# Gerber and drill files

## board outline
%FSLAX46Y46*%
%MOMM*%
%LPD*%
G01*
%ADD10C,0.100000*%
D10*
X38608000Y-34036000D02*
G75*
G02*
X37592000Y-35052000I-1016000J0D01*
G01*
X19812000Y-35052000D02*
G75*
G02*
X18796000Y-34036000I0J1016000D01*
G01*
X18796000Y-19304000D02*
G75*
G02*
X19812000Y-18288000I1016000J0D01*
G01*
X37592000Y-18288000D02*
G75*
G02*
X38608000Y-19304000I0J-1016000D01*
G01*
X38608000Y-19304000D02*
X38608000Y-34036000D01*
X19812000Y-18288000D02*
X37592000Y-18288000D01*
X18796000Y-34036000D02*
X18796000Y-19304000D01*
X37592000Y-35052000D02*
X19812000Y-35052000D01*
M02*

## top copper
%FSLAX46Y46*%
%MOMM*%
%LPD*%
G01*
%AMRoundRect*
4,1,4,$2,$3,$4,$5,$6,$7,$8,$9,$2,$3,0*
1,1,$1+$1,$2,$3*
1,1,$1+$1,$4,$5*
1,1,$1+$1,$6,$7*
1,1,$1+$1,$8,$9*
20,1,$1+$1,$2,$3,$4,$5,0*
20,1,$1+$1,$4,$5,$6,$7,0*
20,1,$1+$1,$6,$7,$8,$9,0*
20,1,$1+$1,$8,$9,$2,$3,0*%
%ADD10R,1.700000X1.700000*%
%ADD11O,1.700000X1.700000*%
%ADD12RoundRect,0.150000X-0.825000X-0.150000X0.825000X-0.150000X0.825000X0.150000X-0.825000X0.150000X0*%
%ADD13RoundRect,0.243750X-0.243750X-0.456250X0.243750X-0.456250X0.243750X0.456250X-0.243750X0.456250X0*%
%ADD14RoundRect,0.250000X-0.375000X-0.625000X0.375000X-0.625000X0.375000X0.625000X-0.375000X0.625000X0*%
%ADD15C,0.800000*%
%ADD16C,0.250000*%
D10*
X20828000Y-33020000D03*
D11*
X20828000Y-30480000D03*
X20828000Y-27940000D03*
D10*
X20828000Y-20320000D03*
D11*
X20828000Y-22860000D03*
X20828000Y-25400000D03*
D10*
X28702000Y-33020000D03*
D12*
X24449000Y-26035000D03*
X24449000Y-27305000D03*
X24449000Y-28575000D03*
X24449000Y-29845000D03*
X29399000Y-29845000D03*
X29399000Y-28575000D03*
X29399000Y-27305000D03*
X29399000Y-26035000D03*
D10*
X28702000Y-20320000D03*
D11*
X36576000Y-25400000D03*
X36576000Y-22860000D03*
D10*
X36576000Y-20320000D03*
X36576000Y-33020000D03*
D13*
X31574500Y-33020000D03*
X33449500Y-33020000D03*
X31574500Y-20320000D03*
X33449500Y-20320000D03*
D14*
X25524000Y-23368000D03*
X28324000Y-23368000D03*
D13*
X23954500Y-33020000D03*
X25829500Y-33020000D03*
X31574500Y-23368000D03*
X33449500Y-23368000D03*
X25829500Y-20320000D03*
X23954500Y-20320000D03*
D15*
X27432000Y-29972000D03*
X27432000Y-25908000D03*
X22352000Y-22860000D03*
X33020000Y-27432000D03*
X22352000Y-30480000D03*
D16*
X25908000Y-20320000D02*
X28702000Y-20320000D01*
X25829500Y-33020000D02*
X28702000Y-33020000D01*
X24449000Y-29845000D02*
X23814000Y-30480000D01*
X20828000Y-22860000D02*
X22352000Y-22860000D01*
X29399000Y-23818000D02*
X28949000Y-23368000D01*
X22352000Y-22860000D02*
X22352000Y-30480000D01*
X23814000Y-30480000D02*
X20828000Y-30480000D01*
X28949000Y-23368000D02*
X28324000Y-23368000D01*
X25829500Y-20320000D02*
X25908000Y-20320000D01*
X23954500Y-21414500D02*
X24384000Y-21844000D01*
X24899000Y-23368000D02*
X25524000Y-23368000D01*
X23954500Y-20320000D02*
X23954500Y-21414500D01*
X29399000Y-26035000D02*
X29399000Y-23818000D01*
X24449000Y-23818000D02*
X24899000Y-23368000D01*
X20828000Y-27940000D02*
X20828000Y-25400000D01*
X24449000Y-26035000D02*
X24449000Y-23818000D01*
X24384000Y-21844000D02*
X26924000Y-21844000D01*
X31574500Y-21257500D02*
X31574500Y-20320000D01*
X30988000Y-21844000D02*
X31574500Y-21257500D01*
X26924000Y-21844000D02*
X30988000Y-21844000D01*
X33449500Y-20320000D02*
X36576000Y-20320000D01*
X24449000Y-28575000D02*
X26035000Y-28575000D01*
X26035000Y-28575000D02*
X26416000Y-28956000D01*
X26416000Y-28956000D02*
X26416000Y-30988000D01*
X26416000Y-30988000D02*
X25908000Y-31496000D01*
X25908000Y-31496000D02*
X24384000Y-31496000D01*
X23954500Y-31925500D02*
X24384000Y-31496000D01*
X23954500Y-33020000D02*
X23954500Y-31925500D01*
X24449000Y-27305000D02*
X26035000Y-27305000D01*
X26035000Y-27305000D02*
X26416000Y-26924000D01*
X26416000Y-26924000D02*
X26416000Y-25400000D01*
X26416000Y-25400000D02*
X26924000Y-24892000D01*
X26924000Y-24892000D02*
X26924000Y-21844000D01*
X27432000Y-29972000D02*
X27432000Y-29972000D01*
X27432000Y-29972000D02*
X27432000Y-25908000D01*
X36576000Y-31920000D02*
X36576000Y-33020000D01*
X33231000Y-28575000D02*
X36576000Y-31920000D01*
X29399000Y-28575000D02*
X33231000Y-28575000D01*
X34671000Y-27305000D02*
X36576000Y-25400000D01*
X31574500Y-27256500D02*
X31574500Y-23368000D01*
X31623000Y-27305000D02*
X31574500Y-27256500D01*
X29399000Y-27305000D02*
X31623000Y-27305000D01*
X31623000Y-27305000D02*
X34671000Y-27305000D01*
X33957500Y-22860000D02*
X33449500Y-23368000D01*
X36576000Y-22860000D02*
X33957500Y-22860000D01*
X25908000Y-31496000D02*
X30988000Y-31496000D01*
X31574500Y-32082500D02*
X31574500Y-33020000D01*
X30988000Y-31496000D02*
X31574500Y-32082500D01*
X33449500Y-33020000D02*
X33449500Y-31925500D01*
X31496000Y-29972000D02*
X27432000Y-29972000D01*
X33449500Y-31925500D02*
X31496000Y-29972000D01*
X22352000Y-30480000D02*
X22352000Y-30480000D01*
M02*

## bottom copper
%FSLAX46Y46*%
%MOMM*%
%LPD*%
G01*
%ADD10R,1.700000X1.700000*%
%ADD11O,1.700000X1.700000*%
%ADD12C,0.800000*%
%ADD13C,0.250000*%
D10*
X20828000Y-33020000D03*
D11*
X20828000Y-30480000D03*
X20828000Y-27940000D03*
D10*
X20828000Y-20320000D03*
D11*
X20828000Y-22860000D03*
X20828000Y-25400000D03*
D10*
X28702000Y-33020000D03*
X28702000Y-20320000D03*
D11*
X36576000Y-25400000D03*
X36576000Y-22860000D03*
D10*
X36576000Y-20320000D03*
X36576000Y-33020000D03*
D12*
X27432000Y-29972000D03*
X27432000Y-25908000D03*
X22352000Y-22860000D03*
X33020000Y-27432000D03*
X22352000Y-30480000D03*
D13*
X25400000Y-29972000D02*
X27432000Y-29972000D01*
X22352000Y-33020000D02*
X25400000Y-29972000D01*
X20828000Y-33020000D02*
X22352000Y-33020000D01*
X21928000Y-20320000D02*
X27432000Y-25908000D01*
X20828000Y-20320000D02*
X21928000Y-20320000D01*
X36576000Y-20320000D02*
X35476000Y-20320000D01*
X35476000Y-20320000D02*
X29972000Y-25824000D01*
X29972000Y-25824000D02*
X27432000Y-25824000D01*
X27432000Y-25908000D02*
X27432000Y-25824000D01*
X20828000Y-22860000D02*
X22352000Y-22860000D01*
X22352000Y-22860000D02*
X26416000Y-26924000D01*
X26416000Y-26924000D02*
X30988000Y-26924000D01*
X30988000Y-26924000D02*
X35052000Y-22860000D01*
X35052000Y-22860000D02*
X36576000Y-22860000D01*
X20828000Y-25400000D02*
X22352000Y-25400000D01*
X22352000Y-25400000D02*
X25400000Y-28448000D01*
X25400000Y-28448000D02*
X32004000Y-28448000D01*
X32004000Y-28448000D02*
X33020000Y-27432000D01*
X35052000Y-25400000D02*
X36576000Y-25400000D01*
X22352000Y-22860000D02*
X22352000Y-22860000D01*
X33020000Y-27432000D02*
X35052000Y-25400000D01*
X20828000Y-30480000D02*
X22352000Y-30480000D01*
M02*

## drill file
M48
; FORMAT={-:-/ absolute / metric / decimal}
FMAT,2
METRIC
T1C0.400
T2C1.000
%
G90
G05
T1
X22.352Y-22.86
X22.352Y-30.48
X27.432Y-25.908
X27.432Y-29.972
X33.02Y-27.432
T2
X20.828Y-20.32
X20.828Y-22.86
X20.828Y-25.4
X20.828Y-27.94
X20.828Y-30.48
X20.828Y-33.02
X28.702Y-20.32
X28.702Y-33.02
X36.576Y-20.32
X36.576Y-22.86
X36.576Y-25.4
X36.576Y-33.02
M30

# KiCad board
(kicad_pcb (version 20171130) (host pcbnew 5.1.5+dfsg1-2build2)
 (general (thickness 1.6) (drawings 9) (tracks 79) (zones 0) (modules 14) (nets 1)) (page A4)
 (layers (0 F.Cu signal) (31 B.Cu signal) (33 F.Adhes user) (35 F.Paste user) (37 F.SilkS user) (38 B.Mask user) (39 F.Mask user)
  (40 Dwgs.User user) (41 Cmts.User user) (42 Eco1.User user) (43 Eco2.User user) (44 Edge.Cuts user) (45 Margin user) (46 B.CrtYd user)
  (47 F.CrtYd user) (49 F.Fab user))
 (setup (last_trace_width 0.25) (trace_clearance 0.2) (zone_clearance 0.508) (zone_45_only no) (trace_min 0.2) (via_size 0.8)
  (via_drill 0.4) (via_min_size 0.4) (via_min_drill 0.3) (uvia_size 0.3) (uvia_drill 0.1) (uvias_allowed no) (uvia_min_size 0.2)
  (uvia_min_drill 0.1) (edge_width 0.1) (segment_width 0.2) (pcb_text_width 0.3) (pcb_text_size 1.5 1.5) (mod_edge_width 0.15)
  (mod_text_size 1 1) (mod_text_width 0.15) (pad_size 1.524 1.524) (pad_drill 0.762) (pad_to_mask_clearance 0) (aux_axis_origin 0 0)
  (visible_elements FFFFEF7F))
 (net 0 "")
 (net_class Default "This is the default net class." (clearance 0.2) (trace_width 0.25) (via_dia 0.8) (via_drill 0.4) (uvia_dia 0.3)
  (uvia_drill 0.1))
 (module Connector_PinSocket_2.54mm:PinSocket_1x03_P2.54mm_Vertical (layer F.Cu) (at 20.828 33.02 180)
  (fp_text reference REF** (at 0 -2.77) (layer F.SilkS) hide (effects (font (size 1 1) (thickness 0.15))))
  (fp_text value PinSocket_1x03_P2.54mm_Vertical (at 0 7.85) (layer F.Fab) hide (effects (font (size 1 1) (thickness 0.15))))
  (pad 1 thru_hole rect (at 0 0 180) (size 1.7 1.7) (drill 1) (layers *.Cu *.Mask))
  (pad 2 thru_hole oval (at 0 2.54 180) (size 1.7 1.7) (drill 1) (layers *.Cu *.Mask))
  (pad 3 thru_hole oval (at 0 5.08 180) (size 1.7 1.7) (drill 1) (layers *.Cu *.Mask)))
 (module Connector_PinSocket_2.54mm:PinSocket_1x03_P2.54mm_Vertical (layer F.Cu) (at 20.828 20.32)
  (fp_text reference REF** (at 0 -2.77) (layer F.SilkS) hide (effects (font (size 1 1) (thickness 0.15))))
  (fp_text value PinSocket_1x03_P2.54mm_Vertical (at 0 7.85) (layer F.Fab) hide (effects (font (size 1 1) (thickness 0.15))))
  (pad 1 thru_hole rect (at 0 0) (size 1.7 1.7) (drill 1) (layers *.Cu *.Mask))
  (pad 2 thru_hole oval (at 0 2.54) (size 1.7 1.7) (drill 1) (layers *.Cu *.Mask))
  (pad 3 thru_hole oval (at 0 5.08) (size 1.7 1.7) (drill 1) (layers *.Cu *.Mask)))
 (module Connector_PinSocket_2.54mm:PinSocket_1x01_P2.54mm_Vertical (layer F.Cu) (at 28.702 33.02)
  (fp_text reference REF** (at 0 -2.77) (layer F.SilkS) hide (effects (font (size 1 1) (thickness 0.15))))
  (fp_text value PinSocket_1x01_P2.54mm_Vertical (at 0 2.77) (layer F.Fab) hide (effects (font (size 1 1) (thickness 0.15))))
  (pad 1 thru_hole rect (at 0 0) (size 1.7 1.7) (drill 1) (layers *.Cu *.Mask)))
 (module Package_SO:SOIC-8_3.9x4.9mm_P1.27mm (layer F.Cu) (at 26.924 27.94)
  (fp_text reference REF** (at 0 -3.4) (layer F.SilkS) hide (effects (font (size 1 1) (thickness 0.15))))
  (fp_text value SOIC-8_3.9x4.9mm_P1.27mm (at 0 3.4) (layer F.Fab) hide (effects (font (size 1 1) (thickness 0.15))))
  (pad 1 smd roundrect (at -2.475 -1.905) (size 1.95 0.6) (layers F.Cu F.Paste F.Mask) (roundrect_rratio 0.25))
  (pad 2 smd roundrect (at -2.475 -0.635) (size 1.95 0.6) (layers F.Cu F.Paste F.Mask) (roundrect_rratio 0.25))
  (pad 3 smd roundrect (at -2.475 0.635) (size 1.95 0.6) (layers F.Cu F.Paste F.Mask) (roundrect_rratio 0.25))
  (pad 4 smd roundrect (at -2.475 1.905) (size 1.95 0.6) (layers F.Cu F.Paste F.Mask) (roundrect_rratio 0.25))
  (pad 5 smd roundrect (at 2.475 1.905) (size 1.95 0.6) (layers F.Cu F.Paste F.Mask) (roundrect_rratio 0.25))
  (pad 6 smd roundrect (at 2.475 0.635) (size 1.95 0.6) (layers F.Cu F.Paste F.Mask) (roundrect_rratio 0.25))
  (pad 7 smd roundrect (at 2.475 -0.635) (size 1.95 0.6) (layers F.Cu F.Paste F.Mask) (roundrect_rratio 0.25))
  (pad 8 smd roundrect (at 2.475 -1.905) (size 1.95 0.6) (layers F.Cu F.Paste F.Mask) (roundrect_rratio 0.25)))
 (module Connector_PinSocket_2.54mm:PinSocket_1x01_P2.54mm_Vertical (layer F.Cu) (at 28.702 20.32)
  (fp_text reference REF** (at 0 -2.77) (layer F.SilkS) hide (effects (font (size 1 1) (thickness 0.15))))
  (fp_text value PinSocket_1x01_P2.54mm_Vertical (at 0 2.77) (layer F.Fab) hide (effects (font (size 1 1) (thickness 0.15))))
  (pad 1 thru_hole rect (at 0 0) (size 1.7 1.7) (drill 1) (layers *.Cu *.Mask)))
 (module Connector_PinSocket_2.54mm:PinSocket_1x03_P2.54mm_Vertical (layer F.Cu) (at 36.576 20.32)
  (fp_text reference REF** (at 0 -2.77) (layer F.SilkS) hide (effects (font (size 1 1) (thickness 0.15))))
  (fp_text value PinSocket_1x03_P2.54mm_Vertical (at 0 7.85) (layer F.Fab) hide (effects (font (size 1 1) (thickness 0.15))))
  (pad 3 thru_hole oval (at 0 5.08) (size 1.7 1.7) (drill 1) (layers *.Cu *.Mask))
  (pad 2 thru_hole oval (at 0 2.54) (size 1.7 1.7) (drill 1) (layers *.Cu *.Mask))
  (pad 1 thru_hole rect (at 0 0) (size 1.7 1.7) (drill 1) (layers *.Cu *.Mask)))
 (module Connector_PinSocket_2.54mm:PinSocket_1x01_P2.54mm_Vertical (layer F.Cu) (at 36.576 33.02)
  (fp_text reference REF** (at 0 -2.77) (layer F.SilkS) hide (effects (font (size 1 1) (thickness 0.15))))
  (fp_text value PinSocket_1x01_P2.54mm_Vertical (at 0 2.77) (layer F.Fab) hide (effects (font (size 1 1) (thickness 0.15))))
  (pad 1 thru_hole rect (at 0 0) (size 1.7 1.7) (drill 1) (layers *.Cu *.Mask)))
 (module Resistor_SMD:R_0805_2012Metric (layer F.Cu) (at 32.512 33.02)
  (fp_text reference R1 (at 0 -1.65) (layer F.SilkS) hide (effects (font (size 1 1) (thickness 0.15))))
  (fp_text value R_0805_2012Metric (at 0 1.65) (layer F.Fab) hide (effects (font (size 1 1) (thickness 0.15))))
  (pad 1 smd roundrect (at -0.9375 0) (size 0.975 1.4) (layers F.Cu F.Paste F.Mask) (roundrect_rratio 0.25))
  (pad 2 smd roundrect (at 0.9375 0) (size 0.975 1.4) (layers F.Cu F.Paste F.Mask) (roundrect_rratio 0.25)))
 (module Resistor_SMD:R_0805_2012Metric (layer F.Cu) (at 32.512 20.32)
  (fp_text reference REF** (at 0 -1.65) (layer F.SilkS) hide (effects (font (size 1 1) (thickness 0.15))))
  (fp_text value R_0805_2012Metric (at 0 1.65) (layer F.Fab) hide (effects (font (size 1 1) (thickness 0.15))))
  (pad 1 smd roundrect (at -0.9375 0) (size 0.975 1.4) (layers F.Cu F.Paste F.Mask) (roundrect_rratio 0.25))
  (pad 2 smd roundrect (at 0.9375 0) (size 0.975 1.4) (layers F.Cu F.Paste F.Mask) (roundrect_rratio 0.25)))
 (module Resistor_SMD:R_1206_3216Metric (layer F.Cu) (at 26.924 23.368)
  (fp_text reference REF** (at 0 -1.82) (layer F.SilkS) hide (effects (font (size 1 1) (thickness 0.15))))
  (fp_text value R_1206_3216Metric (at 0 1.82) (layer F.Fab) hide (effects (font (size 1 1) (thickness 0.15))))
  (pad 1 smd roundrect (at -1.4 0) (size 1.25 1.75) (layers F.Cu F.Paste F.Mask) (roundrect_rratio 0.2))
  (pad 2 smd roundrect (at 1.4 0) (size 1.25 1.75) (layers F.Cu F.Paste F.Mask) (roundrect_rratio 0.2)))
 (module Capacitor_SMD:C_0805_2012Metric (layer F.Cu) (at 24.892 33.02)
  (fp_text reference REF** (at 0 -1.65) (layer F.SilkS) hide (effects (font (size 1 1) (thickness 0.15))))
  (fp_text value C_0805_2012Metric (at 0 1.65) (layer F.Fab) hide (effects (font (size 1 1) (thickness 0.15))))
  (pad 1 smd roundrect (at -0.9375 0) (size 0.975 1.4) (layers F.Cu F.Paste F.Mask) (roundrect_rratio 0.25))
  (pad 2 smd roundrect (at 0.9375 0) (size 0.975 1.4) (layers F.Cu F.Paste F.Mask) (roundrect_rratio 0.25)))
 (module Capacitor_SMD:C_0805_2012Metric (layer F.Cu) (at 32.512 23.368)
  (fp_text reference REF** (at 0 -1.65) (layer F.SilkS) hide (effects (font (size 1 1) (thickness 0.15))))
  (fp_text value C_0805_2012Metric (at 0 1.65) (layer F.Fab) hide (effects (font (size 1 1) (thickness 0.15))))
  (pad 1 smd roundrect (at -0.9375 0) (size 0.975 1.4) (layers F.Cu F.Paste F.Mask) (roundrect_rratio 0.25))
  (pad 2 smd roundrect (at 0.9375 0) (size 0.975 1.4) (layers F.Cu F.Paste F.Mask) (roundrect_rratio 0.25)))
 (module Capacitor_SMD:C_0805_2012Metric (layer F.Cu) (at 24.892 20.32)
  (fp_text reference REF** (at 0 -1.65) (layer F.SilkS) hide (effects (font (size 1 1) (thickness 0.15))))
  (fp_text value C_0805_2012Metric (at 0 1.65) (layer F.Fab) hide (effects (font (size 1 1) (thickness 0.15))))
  (pad 2 smd roundrect (at 0.9375 0) (size 0.975 1.4) (layers F.Cu F.Paste F.Mask) (roundrect_rratio 0.25))
  (pad 1 smd roundrect (at -0.9375 0) (size 0.975 1.4) (layers F.Cu F.Paste F.Mask) (roundrect_rratio 0.25)))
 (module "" (layer F.Cu) (at 33.02 36.83)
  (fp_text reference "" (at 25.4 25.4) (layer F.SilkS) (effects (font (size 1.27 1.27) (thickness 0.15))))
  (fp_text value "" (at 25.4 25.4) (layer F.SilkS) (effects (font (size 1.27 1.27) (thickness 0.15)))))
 (gr_arc (start 37.592 34.036) (end 37.592 35.052) (angle -90) (layer Edge.Cuts) (width 0.1))
 (gr_arc (start 19.812 34.036) (end 18.796 34.036) (angle -90) (layer Edge.Cuts) (width 0.1))
 (gr_arc (start 19.812 19.304) (end 19.812 18.288) (angle -90) (layer Edge.Cuts) (width 0.1))
 (gr_arc (start 37.592 19.304) (end 38.608 19.304) (angle -90) (layer Edge.Cuts) (width 0.1))
 (gr_line (start 38.608 19.304) (end 38.608 34.036) (layer Edge.Cuts) (width 0.1))
 (gr_line (start 19.812 18.288) (end 37.592 18.288) (layer Edge.Cuts) (width 0.1))
 (gr_line (start 18.796 34.036) (end 18.796 19.304) (layer Edge.Cuts) (width 0.1))
 (gr_line (start 37.592 35.052) (end 19.812 35.052) (layer Edge.Cuts) (width 0.1))
 (segment (start 25.908 20.32) (end 28.702 20.32) (width 0.25) (layer F.Cu) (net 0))
 (segment (start 25.8295 33.02) (end 28.702 33.02) (width 0.25) (layer F.Cu) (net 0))
 (segment (start 24.449 29.845) (end 23.814 30.48) (width 0.25) (layer F.Cu) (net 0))
 (segment (start 20.828 22.86) (end 22.352 22.86) (width 0.25) (layer F.Cu) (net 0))
 (segment (start 29.399 23.818) (end 28.949 23.368) (width 0.25) (layer F.Cu) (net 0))
 (segment (start 22.352 22.86) (end 22.352 30.48) (width 0.25) (layer F.Cu) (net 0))
 (segment (start 23.814 30.48) (end 20.828 30.48) (width 0.25) (layer F.Cu) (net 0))
 (segment (start 28.949 23.368) (end 28.324 23.368) (width 0.25) (layer F.Cu) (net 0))
 (segment (start 25.8295 20.32) (end 25.908 20.32) (width 0.25) (layer F.Cu) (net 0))
 (segment (start 23.9545 21.4145) (end 24.384 21.844) (width 0.25) (layer F.Cu) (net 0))
 (segment (start 24.899 23.368) (end 25.524 23.368) (width 0.25) (layer F.Cu) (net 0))
 (segment (start 23.9545 20.32) (end 23.9545 21.4145) (width 0.25) (layer F.Cu) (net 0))
 (segment (start 29.399 26.035) (end 29.399 23.818) (width 0.25) (layer F.Cu) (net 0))
 (segment (start 24.449 23.818) (end 24.899 23.368) (width 0.25) (layer F.Cu) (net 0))
 (segment (start 20.828 27.94) (end 20.828 25.4) (width 0.25) (layer F.Cu) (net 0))
 (segment (start 24.449 26.035) (end 24.449 23.818) (width 0.25) (layer F.Cu) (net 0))
 (segment (start 24.384 21.844) (end 26.924 21.844) (width 0.25) (layer F.Cu) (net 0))
 (segment (start 31.5745 21.2575) (end 31.5745 20.32) (width 0.25) (layer F.Cu) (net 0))
 (segment (start 30.988 21.844) (end 31.5745 21.2575) (width 0.25) (layer F.Cu) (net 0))
 (segment (start 26.924 21.844) (end 30.988 21.844) (width 0.25) (layer F.Cu) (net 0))
 (segment (start 33.4495 20.32) (end 36.576 20.32) (width 0.25) (layer F.Cu) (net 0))
 (segment (start 24.449 28.575) (end 26.035 28.575) (width 0.25) (layer F.Cu) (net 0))
 (segment (start 26.035 28.575) (end 26.416 28.956) (width 0.25) (layer F.Cu) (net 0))
 (segment (start 26.416 28.956) (end 26.416 30.988) (width 0.25) (layer F.Cu) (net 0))
 (segment (start 26.416 30.988) (end 25.908 31.496) (width 0.25) (layer F.Cu) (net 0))
 (segment (start 25.908 31.496) (end 24.384 31.496) (width 0.25) (layer F.Cu) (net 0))
 (segment (start 23.9545 31.9255) (end 24.384 31.496) (width 0.25) (layer F.Cu) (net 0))
 (segment (start 23.9545 33.02) (end 23.9545 31.9255) (width 0.25) (layer F.Cu) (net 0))
 (segment (start 24.449 27.305) (end 26.035 27.305) (width 0.25) (layer F.Cu) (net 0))
 (segment (start 26.035 27.305) (end 26.416 26.924) (width 0.25) (layer F.Cu) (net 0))
 (segment (start 26.416 26.924) (end 26.416 25.4) (width 0.25) (layer F.Cu) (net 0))
 (segment (start 26.416 25.4) (end 26.924 24.892) (width 0.25) (layer F.Cu) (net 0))
 (segment (start 26.924 24.892) (end 26.924 21.844) (width 0.25) (layer F.Cu) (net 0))
 (segment (start 27.432 29.972) (end 27.432 29.972) (width 0.25) (layer F.Cu) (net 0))
 (via (at 27.432 29.972) (size 0.8) (drill 0.4) (layers F.Cu B.Cu) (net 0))
 (segment (start 25.4 29.972) (end 27.432 29.972) (width 0.25) (layer B.Cu) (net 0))
 (segment (start 22.352 33.02) (end 25.4 29.972) (width 0.25) (layer B.Cu) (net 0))
 (segment (start 20.828 33.02) (end 22.352 33.02) (width 0.25) (layer B.Cu) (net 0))
 (segment (start 21.928 20.32) (end 27.432 25.908) (width 0.25) (layer B.Cu) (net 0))
 (segment (start 20.828 20.32) (end 21.928 20.32) (width 0.25) (layer B.Cu) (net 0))
 (segment (start 36.576 20.32) (end 35.476 20.32) (width 0.25) (layer B.Cu) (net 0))
 (segment (start 35.476 20.32) (end 29.972 25.824) (width 0.25) (layer B.Cu) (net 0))
 (segment (start 29.972 25.824) (end 27.432 25.824) (width 0.25) (layer B.Cu) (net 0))
 (segment (start 27.432 25.908) (end 27.432 25.824) (width 0.25) (layer B.Cu) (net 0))
 (via (at 27.432 25.908) (size 0.8) (drill 0.4) (layers F.Cu B.Cu) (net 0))
 (segment (start 27.432 29.972) (end 27.432 25.908) (width 0.25) (layer F.Cu) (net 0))
 (segment (start 36.576 31.92) (end 36.576 33.02) (width 0.25) (layer F.Cu) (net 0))
 (segment (start 33.231 28.575) (end 36.576 31.92) (width 0.25) (layer F.Cu) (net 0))
 (segment (start 29.399 28.575) (end 33.231 28.575) (width 0.25) (layer F.Cu) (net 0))
 (segment (start 20.828 22.86) (end 22.352 22.86) (width 0.25) (layer B.Cu) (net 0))
 (segment (start 22.352 22.86) (end 26.416 26.924) (width 0.25) (layer B.Cu) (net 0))
 (segment (start 26.416 26.924) (end 30.988 26.924) (width 0.25) (layer B.Cu) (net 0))
 (segment (start 30.988 26.924) (end 35.052 22.86) (width 0.25) (layer B.Cu) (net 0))
 (segment (start 35.052 22.86) (end 36.576 22.86) (width 0.25) (layer B.Cu) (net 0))
 (segment (start 20.828 25.4) (end 22.352 25.4) (width 0.25) (layer B.Cu) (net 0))
 (segment (start 22.352 25.4) (end 25.4 28.448) (width 0.25) (layer B.Cu) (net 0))
 (segment (start 25.4 28.448) (end 32.004 28.448) (width 0.25) (layer B.Cu) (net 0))
 (segment (start 32.004 28.448) (end 33.02 27.432) (width 0.25) (layer B.Cu) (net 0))
 (segment (start 35.052 25.4) (end 36.576 25.4) (width 0.25) (layer B.Cu) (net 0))
 (segment (start 34.671 27.305) (end 36.576 25.4) (width 0.25) (layer F.Cu) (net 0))
 (segment (start 31.5745 27.2565) (end 31.5745 23.368) (width 0.25) (layer F.Cu) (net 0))
 (segment (start 31.623 27.305) (end 31.5745 27.2565) (width 0.25) (layer F.Cu) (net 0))
 (segment (start 29.399 27.305) (end 31.623 27.305) (width 0.25) (layer F.Cu) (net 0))
 (segment (start 31.623 27.305) (end 34.671 27.305) (width 0.25) (layer F.Cu) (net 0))
 (segment (start 33.9575 22.86) (end 33.4495 23.368) (width 0.25) (layer F.Cu) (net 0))
 (segment (start 36.576 22.86) (end 33.9575 22.86) (width 0.25) (layer F.Cu) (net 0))
 (segment (start 25.908 31.496) (end 30.988 31.496) (width 0.25) (layer F.Cu) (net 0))
 (segment (start 31.5745 32.0825) (end 31.5745 33.02) (width 0.25) (layer F.Cu) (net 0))
 (segment (start 30.988 31.496) (end 31.5745 32.0825) (width 0.25) (layer F.Cu) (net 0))
 (segment (start 33.4495 33.02) (end 33.4495 31.9255) (width 0.25) (layer F.Cu) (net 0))
 (segment (start 31.496 29.972) (end 27.432 29.972) (width 0.25) (layer F.Cu) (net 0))
 (segment (start 33.4495 31.9255) (end 31.496 29.972) (width 0.25) (layer F.Cu) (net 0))
 (segment (start 22.352 22.86) (end 22.352 22.86) (width 0.25) (layer B.Cu) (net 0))
 (via (at 22.352 22.86) (size 0.8) (drill 0.4) (layers F.Cu B.Cu) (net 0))
 (segment (start 33.02 27.432) (end 35.052 25.4) (width 0.25) (layer B.Cu) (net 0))
 (via (at 33.02 27.432) (size 0.8) (drill 0.4) (layers F.Cu B.Cu) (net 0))
 (segment (start 22.352 30.48) (end 22.352 30.48) (width 0.25) (layer F.Cu) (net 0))
 (via (at 22.352 30.48) (size 0.8) (drill 0.4) (layers F.Cu B.Cu) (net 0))
 (segment (start 20.828 30.48) (end 22.352 30.48) (width 0.25) (layer B.Cu) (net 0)))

